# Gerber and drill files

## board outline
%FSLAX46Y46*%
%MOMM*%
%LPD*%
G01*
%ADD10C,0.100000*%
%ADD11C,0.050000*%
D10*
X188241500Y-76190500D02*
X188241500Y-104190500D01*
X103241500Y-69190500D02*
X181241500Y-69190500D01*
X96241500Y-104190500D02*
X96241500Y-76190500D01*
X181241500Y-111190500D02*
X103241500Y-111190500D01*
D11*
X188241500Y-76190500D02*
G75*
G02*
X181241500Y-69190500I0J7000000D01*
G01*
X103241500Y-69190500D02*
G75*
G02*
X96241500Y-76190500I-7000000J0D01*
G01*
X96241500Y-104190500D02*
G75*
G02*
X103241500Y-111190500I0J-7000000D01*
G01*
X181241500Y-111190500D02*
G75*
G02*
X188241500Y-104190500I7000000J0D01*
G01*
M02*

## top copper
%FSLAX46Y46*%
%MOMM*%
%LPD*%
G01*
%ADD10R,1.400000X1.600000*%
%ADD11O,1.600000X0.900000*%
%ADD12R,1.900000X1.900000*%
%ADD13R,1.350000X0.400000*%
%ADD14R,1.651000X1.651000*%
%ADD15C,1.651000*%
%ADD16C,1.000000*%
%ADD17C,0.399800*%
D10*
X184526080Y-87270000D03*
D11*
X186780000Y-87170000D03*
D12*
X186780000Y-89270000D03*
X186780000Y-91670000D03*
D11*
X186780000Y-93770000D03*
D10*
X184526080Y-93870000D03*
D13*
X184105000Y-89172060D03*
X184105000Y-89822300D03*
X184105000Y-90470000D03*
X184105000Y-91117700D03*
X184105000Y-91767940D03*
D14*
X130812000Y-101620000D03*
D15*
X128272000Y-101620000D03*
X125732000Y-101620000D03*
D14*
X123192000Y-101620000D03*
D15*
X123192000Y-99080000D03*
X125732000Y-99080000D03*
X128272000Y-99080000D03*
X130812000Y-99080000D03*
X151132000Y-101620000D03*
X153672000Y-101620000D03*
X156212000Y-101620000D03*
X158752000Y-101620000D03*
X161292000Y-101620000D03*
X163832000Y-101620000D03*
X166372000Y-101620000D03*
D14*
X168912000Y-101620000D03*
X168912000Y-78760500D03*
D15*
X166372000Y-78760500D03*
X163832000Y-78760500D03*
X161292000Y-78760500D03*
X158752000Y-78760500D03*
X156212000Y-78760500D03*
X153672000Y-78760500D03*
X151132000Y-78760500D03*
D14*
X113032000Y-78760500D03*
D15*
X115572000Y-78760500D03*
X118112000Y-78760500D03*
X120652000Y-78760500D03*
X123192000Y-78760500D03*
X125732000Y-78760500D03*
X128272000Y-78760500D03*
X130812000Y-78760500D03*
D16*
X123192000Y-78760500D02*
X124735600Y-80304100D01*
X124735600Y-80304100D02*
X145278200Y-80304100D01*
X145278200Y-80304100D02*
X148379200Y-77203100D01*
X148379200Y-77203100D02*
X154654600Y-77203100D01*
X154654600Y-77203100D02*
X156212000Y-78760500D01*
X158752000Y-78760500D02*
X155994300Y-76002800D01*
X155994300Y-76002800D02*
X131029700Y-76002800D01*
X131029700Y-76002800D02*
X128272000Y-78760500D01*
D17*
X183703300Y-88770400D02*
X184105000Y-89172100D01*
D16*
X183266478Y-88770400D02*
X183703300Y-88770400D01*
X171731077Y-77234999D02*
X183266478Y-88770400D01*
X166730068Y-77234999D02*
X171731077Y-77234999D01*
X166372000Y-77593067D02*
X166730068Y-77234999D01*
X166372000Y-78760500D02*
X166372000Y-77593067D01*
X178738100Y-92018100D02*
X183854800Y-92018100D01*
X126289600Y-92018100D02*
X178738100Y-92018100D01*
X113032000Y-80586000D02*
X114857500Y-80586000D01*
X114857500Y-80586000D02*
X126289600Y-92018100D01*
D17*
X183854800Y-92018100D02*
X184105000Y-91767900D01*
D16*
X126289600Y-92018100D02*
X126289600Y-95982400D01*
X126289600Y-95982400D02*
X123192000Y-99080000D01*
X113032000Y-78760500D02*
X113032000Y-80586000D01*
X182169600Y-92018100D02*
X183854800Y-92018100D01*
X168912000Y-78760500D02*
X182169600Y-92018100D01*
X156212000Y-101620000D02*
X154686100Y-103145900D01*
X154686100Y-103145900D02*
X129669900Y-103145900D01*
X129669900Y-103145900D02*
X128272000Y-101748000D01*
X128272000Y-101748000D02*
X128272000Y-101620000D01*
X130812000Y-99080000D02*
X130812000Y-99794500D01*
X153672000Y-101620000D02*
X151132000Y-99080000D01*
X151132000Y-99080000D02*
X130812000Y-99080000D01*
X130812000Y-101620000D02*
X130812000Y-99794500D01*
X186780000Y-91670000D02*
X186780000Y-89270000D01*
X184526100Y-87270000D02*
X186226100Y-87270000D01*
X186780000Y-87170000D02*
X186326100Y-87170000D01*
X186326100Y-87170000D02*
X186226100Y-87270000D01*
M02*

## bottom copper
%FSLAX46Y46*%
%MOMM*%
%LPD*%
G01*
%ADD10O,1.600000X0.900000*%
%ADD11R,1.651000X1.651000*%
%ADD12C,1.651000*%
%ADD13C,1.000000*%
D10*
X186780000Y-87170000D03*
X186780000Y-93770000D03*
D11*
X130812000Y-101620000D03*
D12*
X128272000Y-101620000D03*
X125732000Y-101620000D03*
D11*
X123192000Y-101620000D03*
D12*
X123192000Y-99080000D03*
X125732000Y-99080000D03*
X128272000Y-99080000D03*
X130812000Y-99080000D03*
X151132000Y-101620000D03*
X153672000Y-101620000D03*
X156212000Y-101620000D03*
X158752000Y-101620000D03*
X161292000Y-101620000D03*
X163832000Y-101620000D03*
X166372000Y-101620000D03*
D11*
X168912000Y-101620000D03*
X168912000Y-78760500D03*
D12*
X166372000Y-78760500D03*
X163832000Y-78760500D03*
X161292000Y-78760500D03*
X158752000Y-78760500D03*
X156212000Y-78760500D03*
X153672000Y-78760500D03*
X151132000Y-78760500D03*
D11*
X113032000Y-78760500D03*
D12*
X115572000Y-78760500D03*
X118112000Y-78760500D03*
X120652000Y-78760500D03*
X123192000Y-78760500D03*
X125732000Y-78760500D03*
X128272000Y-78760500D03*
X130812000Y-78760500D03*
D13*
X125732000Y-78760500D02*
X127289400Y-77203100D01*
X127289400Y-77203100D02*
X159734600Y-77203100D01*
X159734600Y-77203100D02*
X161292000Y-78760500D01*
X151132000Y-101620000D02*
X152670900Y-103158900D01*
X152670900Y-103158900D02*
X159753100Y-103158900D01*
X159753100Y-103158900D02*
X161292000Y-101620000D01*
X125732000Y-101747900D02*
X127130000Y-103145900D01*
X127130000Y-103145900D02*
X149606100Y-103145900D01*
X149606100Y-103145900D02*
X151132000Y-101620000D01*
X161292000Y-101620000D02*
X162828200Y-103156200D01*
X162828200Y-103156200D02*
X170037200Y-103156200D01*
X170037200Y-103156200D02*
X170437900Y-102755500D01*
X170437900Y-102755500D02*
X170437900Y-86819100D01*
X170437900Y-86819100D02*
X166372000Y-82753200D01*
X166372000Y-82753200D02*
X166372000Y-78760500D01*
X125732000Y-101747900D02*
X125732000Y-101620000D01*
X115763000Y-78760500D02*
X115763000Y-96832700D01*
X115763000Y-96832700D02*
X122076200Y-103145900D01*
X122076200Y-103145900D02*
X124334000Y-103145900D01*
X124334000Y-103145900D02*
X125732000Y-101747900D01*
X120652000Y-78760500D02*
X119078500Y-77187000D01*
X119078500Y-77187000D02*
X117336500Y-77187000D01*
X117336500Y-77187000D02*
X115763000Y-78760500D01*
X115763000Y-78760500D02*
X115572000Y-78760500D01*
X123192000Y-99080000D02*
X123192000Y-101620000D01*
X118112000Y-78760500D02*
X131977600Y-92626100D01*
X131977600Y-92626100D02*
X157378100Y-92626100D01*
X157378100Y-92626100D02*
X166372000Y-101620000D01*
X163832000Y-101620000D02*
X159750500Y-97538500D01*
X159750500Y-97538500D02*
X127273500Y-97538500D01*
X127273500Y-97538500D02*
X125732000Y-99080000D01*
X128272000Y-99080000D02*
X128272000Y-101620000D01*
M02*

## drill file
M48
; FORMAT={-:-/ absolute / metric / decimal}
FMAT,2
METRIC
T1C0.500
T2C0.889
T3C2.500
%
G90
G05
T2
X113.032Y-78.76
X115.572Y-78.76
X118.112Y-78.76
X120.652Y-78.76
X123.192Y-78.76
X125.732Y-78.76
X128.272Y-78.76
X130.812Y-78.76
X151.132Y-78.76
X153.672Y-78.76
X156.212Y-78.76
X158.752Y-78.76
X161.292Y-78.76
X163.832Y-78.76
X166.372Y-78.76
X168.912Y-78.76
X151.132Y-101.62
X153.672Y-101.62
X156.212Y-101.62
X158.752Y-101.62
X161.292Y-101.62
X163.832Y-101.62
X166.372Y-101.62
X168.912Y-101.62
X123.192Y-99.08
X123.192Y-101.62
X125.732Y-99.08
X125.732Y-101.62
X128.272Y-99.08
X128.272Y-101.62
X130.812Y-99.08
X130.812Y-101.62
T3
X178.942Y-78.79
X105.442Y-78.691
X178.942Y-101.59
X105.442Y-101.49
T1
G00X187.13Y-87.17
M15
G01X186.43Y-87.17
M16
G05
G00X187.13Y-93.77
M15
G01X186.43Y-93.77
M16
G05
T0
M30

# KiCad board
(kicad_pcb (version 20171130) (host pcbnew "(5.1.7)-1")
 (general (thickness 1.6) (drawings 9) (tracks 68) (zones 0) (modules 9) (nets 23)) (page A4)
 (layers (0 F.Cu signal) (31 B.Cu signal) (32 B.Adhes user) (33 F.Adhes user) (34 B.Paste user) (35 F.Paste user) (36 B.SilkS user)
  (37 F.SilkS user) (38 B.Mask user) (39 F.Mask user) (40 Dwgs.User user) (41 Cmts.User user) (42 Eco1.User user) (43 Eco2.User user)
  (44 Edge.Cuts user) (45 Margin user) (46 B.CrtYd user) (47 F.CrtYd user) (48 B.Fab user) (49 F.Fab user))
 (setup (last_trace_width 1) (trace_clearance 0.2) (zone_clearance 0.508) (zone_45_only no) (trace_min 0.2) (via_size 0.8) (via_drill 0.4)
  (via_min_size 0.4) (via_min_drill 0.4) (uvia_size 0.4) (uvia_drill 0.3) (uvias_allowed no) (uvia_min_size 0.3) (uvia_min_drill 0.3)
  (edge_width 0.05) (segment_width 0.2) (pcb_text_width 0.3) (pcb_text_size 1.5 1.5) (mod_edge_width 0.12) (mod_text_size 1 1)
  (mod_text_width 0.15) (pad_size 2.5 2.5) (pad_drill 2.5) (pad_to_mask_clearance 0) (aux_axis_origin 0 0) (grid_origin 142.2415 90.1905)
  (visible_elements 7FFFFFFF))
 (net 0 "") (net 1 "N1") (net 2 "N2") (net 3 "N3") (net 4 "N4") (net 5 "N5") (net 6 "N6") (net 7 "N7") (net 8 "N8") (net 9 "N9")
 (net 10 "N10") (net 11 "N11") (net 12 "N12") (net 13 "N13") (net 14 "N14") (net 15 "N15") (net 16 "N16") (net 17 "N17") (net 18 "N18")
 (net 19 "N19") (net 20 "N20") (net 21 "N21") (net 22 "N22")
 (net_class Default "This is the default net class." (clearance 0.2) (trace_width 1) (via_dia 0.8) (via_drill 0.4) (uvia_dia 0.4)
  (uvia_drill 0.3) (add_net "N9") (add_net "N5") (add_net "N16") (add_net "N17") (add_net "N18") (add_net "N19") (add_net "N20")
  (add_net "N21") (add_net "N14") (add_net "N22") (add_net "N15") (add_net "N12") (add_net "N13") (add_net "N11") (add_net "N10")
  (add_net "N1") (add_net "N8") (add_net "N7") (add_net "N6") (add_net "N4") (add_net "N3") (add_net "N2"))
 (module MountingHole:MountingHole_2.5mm (layer F.Cu) (at 105.442 78.6905)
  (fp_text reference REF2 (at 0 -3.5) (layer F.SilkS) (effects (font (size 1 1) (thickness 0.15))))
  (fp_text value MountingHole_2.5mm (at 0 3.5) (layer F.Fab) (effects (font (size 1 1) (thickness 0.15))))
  (pad 1 np_thru_hole circle (at 0 0) (size 2.5 2.5) (drill 2.5) (layers *.Cu *.Mask)))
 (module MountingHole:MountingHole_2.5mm (layer F.Cu) (at 105.442 101.49)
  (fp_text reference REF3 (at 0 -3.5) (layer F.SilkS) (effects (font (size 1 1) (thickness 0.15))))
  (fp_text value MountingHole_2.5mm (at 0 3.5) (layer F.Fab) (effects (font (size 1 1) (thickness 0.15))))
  (pad 1 np_thru_hole circle (at 0 0) (size 2.5 2.5) (drill 2.5) (layers *.Cu *.Mask)))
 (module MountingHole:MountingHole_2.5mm (layer F.Cu) (at 178.942 78.7905)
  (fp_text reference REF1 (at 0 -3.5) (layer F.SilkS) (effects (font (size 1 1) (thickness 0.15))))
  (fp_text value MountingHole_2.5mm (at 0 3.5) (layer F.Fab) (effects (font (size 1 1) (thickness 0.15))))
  (pad 1 np_thru_hole circle (at 0 0) (size 2.5 2.5) (drill 2.5) (layers *.Cu *.Mask)))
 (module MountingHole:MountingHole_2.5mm (layer F.Cu) (at 178.942 101.59)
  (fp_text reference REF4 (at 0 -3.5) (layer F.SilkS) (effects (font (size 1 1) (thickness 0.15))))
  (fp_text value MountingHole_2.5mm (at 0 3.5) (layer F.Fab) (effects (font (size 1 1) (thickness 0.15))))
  (pad 1 np_thru_hole circle (at 0 0) (size 2.5 2.5) (drill 2.5) (layers *.Cu *.Mask)))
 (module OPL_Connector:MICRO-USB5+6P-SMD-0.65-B (layer F.Cu) (at 186.78 90.47 90)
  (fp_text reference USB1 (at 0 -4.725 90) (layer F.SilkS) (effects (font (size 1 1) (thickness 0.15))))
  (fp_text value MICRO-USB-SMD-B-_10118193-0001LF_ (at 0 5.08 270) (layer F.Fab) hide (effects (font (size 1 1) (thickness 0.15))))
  (pad 11 smd rect (at 3.2 -2.25392 180) (size 1.4 1.6) (layers F.Cu F.Paste F.Mask) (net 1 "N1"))
  (pad 10 thru_hole oval (at 3.3 0 270) (size 0.9 1.6) (drill oval 0.5 1.2) (layers *.Cu *.Mask) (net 1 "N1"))
  (pad 9 smd rect (at 1.2 0 90) (size 1.9 1.9) (layers F.Cu F.Paste F.Mask) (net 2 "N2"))
  (pad 8 smd rect (at -1.2 0 90) (size 1.9 1.9) (layers F.Cu F.Paste F.Mask) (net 2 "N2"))
  (pad 7 thru_hole oval (at -3.3 0 270) (size 0.9 1.6) (drill oval 0.5 1.2) (layers *.Cu *.Mask) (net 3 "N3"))
  (pad 6 smd rect (at -3.4 -2.25392 180) (size 1.4 1.6) (layers F.Cu F.Paste F.Mask) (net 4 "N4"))
  (pad 5 smd rect (at 1.29794 -2.675 270) (size 0.4 1.35) (layers F.Cu F.Paste F.Mask) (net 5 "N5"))
  (pad 4 smd rect (at 0.6477 -2.675 270) (size 0.4 1.35) (layers F.Cu F.Paste F.Mask) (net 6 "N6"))
  (pad 3 smd rect (at 0 -2.675 270) (size 0.4 1.35) (layers F.Cu F.Paste F.Mask) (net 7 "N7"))
  (pad 2 smd rect (at -0.6477 -2.675 270) (size 0.4 1.35) (layers F.Cu F.Paste F.Mask) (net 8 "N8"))
  (pad 1 smd rect (at -1.29794 -2.675 270) (size 0.4 1.35) (layers F.Cu F.Paste F.Mask) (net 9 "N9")))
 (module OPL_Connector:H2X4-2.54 (layer F.Cu) (at 127.002 100.35 180)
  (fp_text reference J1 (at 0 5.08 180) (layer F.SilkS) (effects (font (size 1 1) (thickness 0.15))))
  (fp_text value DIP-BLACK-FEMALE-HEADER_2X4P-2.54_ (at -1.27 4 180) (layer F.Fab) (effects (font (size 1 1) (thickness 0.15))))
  (pad 4 thru_hole rect (at -3.81 -1.27 270) (size 1.651 1.651) (drill 0.889) (layers *.Cu *.Mask) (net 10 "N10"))
  (pad 3 thru_hole circle (at -1.27 -1.27 270) (size 1.651 1.651) (drill 0.889) (layers *.Cu *.Mask) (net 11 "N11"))
  (pad 2 thru_hole circle (at 1.27 -1.27 270) (size 1.651 1.651) (drill 0.889) (layers *.Cu *.Mask) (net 5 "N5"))
  (pad 1 thru_hole rect (at 3.81 -1.27 270) (size 1.651 1.651) (drill 0.889) (layers *.Cu *.Mask) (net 9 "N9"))
  (pad 8 thru_hole circle (at 3.81 1.27 270) (size 1.651 1.651) (drill 0.889) (layers *.Cu *.Mask) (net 9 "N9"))
  (pad 7 thru_hole circle (at 1.27 1.27 270) (size 1.651 1.651) (drill 0.889) (layers *.Cu *.Mask) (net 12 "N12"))
  (pad 6 thru_hole circle (at -1.27 1.27 270) (size 1.651 1.651) (drill 0.889) (layers *.Cu *.Mask) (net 11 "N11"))
  (pad 5 thru_hole circle (at -3.81 1.27 270) (size 1.651 1.651) (drill 0.889) (layers *.Cu *.Mask) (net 10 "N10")))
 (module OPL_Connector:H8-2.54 (layer F.Cu) (at 160.022 101.62)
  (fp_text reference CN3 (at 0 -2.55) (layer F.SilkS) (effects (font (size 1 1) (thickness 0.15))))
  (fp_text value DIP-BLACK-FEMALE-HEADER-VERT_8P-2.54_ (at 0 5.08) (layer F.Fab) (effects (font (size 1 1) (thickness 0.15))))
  (pad 8 thru_hole circle (at -8.89 0 270) (size 1.651 1.651) (drill 0.889) (layers *.Cu *.Mask) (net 5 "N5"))
  (pad 7 thru_hole circle (at -6.35 0 270) (size 1.651 1.651) (drill 0.889) (layers *.Cu *.Mask) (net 10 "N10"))
  (pad 6 thru_hole circle (at -3.81 0 270) (size 1.651 1.651) (drill 0.889) (layers *.Cu *.Mask) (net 11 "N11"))
  (pad 5 thru_hole circle (at -1.27 0 270) (size 1.651 1.651) (drill 0.889) (layers *.Cu *.Mask) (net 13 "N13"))
  (pad 4 thru_hole circle (at 1.27 0 270) (size 1.651 1.651) (drill 0.889) (layers *.Cu *.Mask) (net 5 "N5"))
  (pad 3 thru_hole circle (at 3.81 0 270) (size 1.651 1.651) (drill 0.889) (layers *.Cu *.Mask) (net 12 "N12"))
  (pad 2 thru_hole circle (at 6.35 0 270) (size 1.651 1.651) (drill 0.889) (layers *.Cu *.Mask) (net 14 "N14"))
  (pad 1 thru_hole rect (at 8.89 0 270) (size 1.651 1.651) (drill 0.889) (layers *.Cu *.Mask) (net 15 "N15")))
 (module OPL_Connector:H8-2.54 (layer F.Cu) (at 160.022 78.7605)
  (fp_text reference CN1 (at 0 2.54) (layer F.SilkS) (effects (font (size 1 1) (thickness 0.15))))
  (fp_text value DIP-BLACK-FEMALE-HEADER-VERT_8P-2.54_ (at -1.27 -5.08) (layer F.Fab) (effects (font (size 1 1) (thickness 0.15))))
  (pad 1 thru_hole rect (at 8.89 0 270) (size 1.651 1.651) (drill 0.889) (layers *.Cu *.Mask) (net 9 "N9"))
  (pad 2 thru_hole circle (at 6.35 0 270) (size 1.651 1.651) (drill 0.889) (layers *.Cu *.Mask) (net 5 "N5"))
  (pad 3 thru_hole circle (at 3.81 0 270) (size 1.651 1.651) (drill 0.889) (layers *.Cu *.Mask) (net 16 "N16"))
  (pad 4 thru_hole circle (at 1.27 0 270) (size 1.651 1.651) (drill 0.889) (layers *.Cu *.Mask) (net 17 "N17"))
  (pad 5 thru_hole circle (at -1.27 0 270) (size 1.651 1.651) (drill 0.889) (layers *.Cu *.Mask) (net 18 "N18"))
  (pad 6 thru_hole circle (at -3.81 0 270) (size 1.651 1.651) (drill 0.889) (layers *.Cu *.Mask) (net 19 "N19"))
  (pad 7 thru_hole circle (at -6.35 0 270) (size 1.651 1.651) (drill 0.889) (layers *.Cu *.Mask) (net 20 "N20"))
  (pad 8 thru_hole circle (at -8.89 0 270) (size 1.651 1.651) (drill 0.889) (layers *.Cu *.Mask) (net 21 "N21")))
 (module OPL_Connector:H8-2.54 (layer F.Cu) (at 121.922 78.7605 180)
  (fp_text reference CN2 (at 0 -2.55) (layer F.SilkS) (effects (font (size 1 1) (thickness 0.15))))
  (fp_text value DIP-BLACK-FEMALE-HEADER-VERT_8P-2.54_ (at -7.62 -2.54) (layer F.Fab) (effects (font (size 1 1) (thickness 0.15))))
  (pad 1 thru_hole rect (at 8.89 0 90) (size 1.651 1.651) (drill 0.889) (layers *.Cu *.Mask) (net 9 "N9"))
  (pad 2 thru_hole circle (at 6.35 0 90) (size 1.651 1.651) (drill 0.889) (layers *.Cu *.Mask) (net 5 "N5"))
  (pad 3 thru_hole circle (at 3.81 0 90) (size 1.651 1.651) (drill 0.889) (layers *.Cu *.Mask) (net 14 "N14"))
  (pad 4 thru_hole circle (at 1.27 0 90) (size 1.651 1.651) (drill 0.889) (layers *.Cu *.Mask) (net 5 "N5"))
  (pad 5 thru_hole circle (at -1.27 0 90) (size 1.651 1.651) (drill 0.889) (layers *.Cu *.Mask) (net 19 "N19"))
  (pad 6 thru_hole circle (at -3.81 0 90) (size 1.651 1.651) (drill 0.889) (layers *.Cu *.Mask) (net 17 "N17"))
  (pad 7 thru_hole circle (at -6.35 0 90) (size 1.651 1.651) (drill 0.889) (layers *.Cu *.Mask) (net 18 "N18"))
  (pad 8 thru_hole circle (at -8.89 0 90) (size 1.651 1.651) (drill 0.889) (layers *.Cu *.Mask) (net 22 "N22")))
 (gr_line (start 188.2415 76.1905) (end 188.2415 104.1905) (layer Edge.Cuts) (width 0.1))
 (gr_line (start 103.2415 69.1905) (end 181.2415 69.1905) (layer Edge.Cuts) (width 0.1))
 (gr_line (start 96.2415 104.1905) (end 96.2415 76.1905) (layer Edge.Cuts) (width 0.1))
 (gr_line (start 181.2415 111.1905) (end 103.2415 111.1905) (layer Edge.Cuts) (width 0.1))
 (gr_arc (start 188.2415 69.1905) (end 181.2415 69.1905) (angle -90) (layer Edge.Cuts) (width 0.05))
 (gr_arc (start 96.2415 69.1905) (end 96.2415 76.1905) (angle -90) (layer Edge.Cuts) (width 0.05))
 (gr_arc (start 96.2415 111.1905) (end 103.2415 111.1905) (angle -90) (layer Edge.Cuts) (width 0.05))
 (gr_arc (start 188.2415 111.1905) (end 188.2415 104.1905) (angle -90) (layer Edge.Cuts) (width 0.05))
 (segment (start 123.192 78.7605) (end 124.7356 80.3041) (width 1) (layer F.Cu) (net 19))
 (segment (start 124.7356 80.3041) (end 145.2782 80.3041) (width 1) (layer F.Cu) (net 19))
 (segment (start 145.2782 80.3041) (end 148.3792 77.2031) (width 1) (layer F.Cu) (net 19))
 (segment (start 148.3792 77.2031) (end 154.6546 77.2031) (width 1) (layer F.Cu) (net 19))
 (segment (start 154.6546 77.2031) (end 156.212 78.7605) (width 1) (layer F.Cu) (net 19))
 (segment (start 158.752 78.7605) (end 155.9943 76.0028) (width 1) (layer F.Cu) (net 18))
 (segment (start 155.9943 76.0028) (end 131.0297 76.0028) (width 1) (layer F.Cu) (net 18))
 (segment (start 131.0297 76.0028) (end 128.272 78.7605) (width 1) (layer F.Cu) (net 18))
 (segment (start 125.732 78.7605) (end 127.2894 77.2031) (width 1) (layer B.Cu) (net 17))
 (segment (start 127.2894 77.2031) (end 159.7346 77.2031) (width 1) (layer B.Cu) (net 17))
 (segment (start 159.7346 77.2031) (end 161.292 78.7605) (width 1) (layer B.Cu) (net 17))
 (segment (start 151.132 101.62) (end 152.6709 103.1589) (width 1) (layer B.Cu) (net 5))
 (segment (start 152.6709 103.1589) (end 159.7531 103.1589) (width 1) (layer B.Cu) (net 5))
 (segment (start 159.7531 103.1589) (end 161.292 101.62) (width 1) (layer B.Cu) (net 5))
 (segment (start 125.732 101.7479) (end 127.13 103.1459) (width 1) (layer B.Cu) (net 5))
 (segment (start 127.13 103.1459) (end 149.6061 103.1459) (width 1) (layer B.Cu) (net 5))
 (segment (start 149.6061 103.1459) (end 151.132 101.62) (width 1) (layer B.Cu) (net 5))
 (segment (start 161.292 101.62) (end 162.8282 103.1562) (width 1) (layer B.Cu) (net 5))
 (segment (start 162.8282 103.1562) (end 170.0372 103.1562) (width 1) (layer B.Cu) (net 5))
 (segment (start 170.0372 103.1562) (end 170.4379 102.7555) (width 1) (layer B.Cu) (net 5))
 (segment (start 170.4379 102.7555) (end 170.4379 86.8191) (width 1) (layer B.Cu) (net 5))
 (segment (start 170.4379 86.8191) (end 166.372 82.7532) (width 1) (layer B.Cu) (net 5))
 (segment (start 166.372 82.7532) (end 166.372 78.7605) (width 1) (layer B.Cu) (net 5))
 (segment (start 125.732 101.7479) (end 125.732 101.62) (width 1) (layer B.Cu) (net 5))
 (segment (start 115.763 78.7605) (end 115.763 96.8327) (width 1) (layer B.Cu) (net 5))
 (segment (start 115.763 96.8327) (end 122.0762 103.1459) (width 1) (layer B.Cu) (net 5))
 (segment (start 122.0762 103.1459) (end 124.334 103.1459) (width 1) (layer B.Cu) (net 5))
 (segment (start 124.334 103.1459) (end 125.732 101.7479) (width 1) (layer B.Cu) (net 5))
 (segment (start 120.652 78.7605) (end 119.0785 77.187) (width 1) (layer B.Cu) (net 5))
 (segment (start 119.0785 77.187) (end 117.3365 77.187) (width 1) (layer B.Cu) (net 5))
 (segment (start 117.3365 77.187) (end 115.763 78.7605) (width 1) (layer B.Cu) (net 5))
 (segment (start 115.763 78.7605) (end 115.572 78.7605) (width 1) (layer B.Cu) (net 5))
 (segment (start 183.7033 88.7704) (end 184.105 89.1721) (width 0.3998) (layer F.Cu) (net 5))
 (segment (start 183.266478 88.7704) (end 183.7033 88.7704) (width 1) (layer F.Cu) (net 5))
 (segment (start 171.731077 77.234999) (end 183.266478 88.7704) (width 1) (layer F.Cu) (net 5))
 (segment (start 166.730068 77.234999) (end 171.731077 77.234999) (width 1) (layer F.Cu) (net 5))
 (segment (start 166.372 77.593067) (end 166.730068 77.234999) (width 1) (layer F.Cu) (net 5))
 (segment (start 166.372 78.7605) (end 166.372 77.593067) (width 1) (layer F.Cu) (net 5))
 (segment (start 178.7381 92.0181) (end 183.8548 92.0181) (width 1) (layer F.Cu) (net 9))
 (segment (start 126.2896 92.0181) (end 178.7381 92.0181) (width 1) (layer F.Cu) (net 9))
 (segment (start 113.032 80.586) (end 114.8575 80.586) (width 1) (layer F.Cu) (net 9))
 (segment (start 114.8575 80.586) (end 126.2896 92.0181) (width 1) (layer F.Cu) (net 9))
 (segment (start 183.8548 92.0181) (end 184.105 91.7679) (width 0.3998) (layer F.Cu) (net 9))
 (segment (start 126.2896 92.0181) (end 126.2896 95.9824) (width 1) (layer F.Cu) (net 9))
 (segment (start 126.2896 95.9824) (end 123.192 99.08) (width 1) (layer F.Cu) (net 9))
 (segment (start 113.032 78.7605) (end 113.032 80.586) (width 1) (layer F.Cu) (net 9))
 (segment (start 123.192 99.08) (end 123.192 101.62) (width 1) (layer B.Cu) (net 9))
 (segment (start 182.1696 92.0181) (end 183.8548 92.0181) (width 1) (layer F.Cu) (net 9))
 (segment (start 168.912 78.7605) (end 182.1696 92.0181) (width 1) (layer F.Cu) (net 9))
 (segment (start 118.112 78.7605) (end 131.9776 92.6261) (width 1) (layer B.Cu) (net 14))
 (segment (start 131.9776 92.6261) (end 157.3781 92.6261) (width 1) (layer B.Cu) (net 14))
 (segment (start 157.3781 92.6261) (end 166.372 101.62) (width 1) (layer B.Cu) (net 14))
 (segment (start 163.832 101.62) (end 159.7505 97.5385) (width 1) (layer B.Cu) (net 12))
 (segment (start 159.7505 97.5385) (end 127.2735 97.5385) (width 1) (layer B.Cu) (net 12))
 (segment (start 127.2735 97.5385) (end 125.732 99.08) (width 1) (layer B.Cu) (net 12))
 (segment (start 156.212 101.62) (end 154.6861 103.1459) (width 1) (layer F.Cu) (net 11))
 (segment (start 154.6861 103.1459) (end 129.6699 103.1459) (width 1) (layer F.Cu) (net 11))
 (segment (start 129.6699 103.1459) (end 128.272 101.748) (width 1) (layer F.Cu) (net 11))
 (segment (start 128.272 101.748) (end 128.272 101.62) (width 1) (layer F.Cu) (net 11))
 (segment (start 128.272 99.08) (end 128.272 101.62) (width 1) (layer B.Cu) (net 11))
 (segment (start 130.812 99.08) (end 130.812 99.7945) (width 1) (layer F.Cu) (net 10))
 (segment (start 153.672 101.62) (end 151.132 99.08) (width 1) (layer F.Cu) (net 10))
 (segment (start 151.132 99.08) (end 130.812 99.08) (width 1) (layer F.Cu) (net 10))
 (segment (start 130.812 101.62) (end 130.812 99.7945) (width 1) (layer F.Cu) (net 10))
 (segment (start 186.78 91.67) (end 186.78 89.27) (width 1) (layer F.Cu) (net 2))
 (segment (start 184.5261 87.27) (end 186.2261 87.27) (width 1) (layer F.Cu) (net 1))
 (segment (start 186.78 87.17) (end 186.3261 87.17) (width 1) (layer F.Cu) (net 1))
 (segment (start 186.3261 87.17) (end 186.2261 87.27) (width 1) (layer F.Cu) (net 1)))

